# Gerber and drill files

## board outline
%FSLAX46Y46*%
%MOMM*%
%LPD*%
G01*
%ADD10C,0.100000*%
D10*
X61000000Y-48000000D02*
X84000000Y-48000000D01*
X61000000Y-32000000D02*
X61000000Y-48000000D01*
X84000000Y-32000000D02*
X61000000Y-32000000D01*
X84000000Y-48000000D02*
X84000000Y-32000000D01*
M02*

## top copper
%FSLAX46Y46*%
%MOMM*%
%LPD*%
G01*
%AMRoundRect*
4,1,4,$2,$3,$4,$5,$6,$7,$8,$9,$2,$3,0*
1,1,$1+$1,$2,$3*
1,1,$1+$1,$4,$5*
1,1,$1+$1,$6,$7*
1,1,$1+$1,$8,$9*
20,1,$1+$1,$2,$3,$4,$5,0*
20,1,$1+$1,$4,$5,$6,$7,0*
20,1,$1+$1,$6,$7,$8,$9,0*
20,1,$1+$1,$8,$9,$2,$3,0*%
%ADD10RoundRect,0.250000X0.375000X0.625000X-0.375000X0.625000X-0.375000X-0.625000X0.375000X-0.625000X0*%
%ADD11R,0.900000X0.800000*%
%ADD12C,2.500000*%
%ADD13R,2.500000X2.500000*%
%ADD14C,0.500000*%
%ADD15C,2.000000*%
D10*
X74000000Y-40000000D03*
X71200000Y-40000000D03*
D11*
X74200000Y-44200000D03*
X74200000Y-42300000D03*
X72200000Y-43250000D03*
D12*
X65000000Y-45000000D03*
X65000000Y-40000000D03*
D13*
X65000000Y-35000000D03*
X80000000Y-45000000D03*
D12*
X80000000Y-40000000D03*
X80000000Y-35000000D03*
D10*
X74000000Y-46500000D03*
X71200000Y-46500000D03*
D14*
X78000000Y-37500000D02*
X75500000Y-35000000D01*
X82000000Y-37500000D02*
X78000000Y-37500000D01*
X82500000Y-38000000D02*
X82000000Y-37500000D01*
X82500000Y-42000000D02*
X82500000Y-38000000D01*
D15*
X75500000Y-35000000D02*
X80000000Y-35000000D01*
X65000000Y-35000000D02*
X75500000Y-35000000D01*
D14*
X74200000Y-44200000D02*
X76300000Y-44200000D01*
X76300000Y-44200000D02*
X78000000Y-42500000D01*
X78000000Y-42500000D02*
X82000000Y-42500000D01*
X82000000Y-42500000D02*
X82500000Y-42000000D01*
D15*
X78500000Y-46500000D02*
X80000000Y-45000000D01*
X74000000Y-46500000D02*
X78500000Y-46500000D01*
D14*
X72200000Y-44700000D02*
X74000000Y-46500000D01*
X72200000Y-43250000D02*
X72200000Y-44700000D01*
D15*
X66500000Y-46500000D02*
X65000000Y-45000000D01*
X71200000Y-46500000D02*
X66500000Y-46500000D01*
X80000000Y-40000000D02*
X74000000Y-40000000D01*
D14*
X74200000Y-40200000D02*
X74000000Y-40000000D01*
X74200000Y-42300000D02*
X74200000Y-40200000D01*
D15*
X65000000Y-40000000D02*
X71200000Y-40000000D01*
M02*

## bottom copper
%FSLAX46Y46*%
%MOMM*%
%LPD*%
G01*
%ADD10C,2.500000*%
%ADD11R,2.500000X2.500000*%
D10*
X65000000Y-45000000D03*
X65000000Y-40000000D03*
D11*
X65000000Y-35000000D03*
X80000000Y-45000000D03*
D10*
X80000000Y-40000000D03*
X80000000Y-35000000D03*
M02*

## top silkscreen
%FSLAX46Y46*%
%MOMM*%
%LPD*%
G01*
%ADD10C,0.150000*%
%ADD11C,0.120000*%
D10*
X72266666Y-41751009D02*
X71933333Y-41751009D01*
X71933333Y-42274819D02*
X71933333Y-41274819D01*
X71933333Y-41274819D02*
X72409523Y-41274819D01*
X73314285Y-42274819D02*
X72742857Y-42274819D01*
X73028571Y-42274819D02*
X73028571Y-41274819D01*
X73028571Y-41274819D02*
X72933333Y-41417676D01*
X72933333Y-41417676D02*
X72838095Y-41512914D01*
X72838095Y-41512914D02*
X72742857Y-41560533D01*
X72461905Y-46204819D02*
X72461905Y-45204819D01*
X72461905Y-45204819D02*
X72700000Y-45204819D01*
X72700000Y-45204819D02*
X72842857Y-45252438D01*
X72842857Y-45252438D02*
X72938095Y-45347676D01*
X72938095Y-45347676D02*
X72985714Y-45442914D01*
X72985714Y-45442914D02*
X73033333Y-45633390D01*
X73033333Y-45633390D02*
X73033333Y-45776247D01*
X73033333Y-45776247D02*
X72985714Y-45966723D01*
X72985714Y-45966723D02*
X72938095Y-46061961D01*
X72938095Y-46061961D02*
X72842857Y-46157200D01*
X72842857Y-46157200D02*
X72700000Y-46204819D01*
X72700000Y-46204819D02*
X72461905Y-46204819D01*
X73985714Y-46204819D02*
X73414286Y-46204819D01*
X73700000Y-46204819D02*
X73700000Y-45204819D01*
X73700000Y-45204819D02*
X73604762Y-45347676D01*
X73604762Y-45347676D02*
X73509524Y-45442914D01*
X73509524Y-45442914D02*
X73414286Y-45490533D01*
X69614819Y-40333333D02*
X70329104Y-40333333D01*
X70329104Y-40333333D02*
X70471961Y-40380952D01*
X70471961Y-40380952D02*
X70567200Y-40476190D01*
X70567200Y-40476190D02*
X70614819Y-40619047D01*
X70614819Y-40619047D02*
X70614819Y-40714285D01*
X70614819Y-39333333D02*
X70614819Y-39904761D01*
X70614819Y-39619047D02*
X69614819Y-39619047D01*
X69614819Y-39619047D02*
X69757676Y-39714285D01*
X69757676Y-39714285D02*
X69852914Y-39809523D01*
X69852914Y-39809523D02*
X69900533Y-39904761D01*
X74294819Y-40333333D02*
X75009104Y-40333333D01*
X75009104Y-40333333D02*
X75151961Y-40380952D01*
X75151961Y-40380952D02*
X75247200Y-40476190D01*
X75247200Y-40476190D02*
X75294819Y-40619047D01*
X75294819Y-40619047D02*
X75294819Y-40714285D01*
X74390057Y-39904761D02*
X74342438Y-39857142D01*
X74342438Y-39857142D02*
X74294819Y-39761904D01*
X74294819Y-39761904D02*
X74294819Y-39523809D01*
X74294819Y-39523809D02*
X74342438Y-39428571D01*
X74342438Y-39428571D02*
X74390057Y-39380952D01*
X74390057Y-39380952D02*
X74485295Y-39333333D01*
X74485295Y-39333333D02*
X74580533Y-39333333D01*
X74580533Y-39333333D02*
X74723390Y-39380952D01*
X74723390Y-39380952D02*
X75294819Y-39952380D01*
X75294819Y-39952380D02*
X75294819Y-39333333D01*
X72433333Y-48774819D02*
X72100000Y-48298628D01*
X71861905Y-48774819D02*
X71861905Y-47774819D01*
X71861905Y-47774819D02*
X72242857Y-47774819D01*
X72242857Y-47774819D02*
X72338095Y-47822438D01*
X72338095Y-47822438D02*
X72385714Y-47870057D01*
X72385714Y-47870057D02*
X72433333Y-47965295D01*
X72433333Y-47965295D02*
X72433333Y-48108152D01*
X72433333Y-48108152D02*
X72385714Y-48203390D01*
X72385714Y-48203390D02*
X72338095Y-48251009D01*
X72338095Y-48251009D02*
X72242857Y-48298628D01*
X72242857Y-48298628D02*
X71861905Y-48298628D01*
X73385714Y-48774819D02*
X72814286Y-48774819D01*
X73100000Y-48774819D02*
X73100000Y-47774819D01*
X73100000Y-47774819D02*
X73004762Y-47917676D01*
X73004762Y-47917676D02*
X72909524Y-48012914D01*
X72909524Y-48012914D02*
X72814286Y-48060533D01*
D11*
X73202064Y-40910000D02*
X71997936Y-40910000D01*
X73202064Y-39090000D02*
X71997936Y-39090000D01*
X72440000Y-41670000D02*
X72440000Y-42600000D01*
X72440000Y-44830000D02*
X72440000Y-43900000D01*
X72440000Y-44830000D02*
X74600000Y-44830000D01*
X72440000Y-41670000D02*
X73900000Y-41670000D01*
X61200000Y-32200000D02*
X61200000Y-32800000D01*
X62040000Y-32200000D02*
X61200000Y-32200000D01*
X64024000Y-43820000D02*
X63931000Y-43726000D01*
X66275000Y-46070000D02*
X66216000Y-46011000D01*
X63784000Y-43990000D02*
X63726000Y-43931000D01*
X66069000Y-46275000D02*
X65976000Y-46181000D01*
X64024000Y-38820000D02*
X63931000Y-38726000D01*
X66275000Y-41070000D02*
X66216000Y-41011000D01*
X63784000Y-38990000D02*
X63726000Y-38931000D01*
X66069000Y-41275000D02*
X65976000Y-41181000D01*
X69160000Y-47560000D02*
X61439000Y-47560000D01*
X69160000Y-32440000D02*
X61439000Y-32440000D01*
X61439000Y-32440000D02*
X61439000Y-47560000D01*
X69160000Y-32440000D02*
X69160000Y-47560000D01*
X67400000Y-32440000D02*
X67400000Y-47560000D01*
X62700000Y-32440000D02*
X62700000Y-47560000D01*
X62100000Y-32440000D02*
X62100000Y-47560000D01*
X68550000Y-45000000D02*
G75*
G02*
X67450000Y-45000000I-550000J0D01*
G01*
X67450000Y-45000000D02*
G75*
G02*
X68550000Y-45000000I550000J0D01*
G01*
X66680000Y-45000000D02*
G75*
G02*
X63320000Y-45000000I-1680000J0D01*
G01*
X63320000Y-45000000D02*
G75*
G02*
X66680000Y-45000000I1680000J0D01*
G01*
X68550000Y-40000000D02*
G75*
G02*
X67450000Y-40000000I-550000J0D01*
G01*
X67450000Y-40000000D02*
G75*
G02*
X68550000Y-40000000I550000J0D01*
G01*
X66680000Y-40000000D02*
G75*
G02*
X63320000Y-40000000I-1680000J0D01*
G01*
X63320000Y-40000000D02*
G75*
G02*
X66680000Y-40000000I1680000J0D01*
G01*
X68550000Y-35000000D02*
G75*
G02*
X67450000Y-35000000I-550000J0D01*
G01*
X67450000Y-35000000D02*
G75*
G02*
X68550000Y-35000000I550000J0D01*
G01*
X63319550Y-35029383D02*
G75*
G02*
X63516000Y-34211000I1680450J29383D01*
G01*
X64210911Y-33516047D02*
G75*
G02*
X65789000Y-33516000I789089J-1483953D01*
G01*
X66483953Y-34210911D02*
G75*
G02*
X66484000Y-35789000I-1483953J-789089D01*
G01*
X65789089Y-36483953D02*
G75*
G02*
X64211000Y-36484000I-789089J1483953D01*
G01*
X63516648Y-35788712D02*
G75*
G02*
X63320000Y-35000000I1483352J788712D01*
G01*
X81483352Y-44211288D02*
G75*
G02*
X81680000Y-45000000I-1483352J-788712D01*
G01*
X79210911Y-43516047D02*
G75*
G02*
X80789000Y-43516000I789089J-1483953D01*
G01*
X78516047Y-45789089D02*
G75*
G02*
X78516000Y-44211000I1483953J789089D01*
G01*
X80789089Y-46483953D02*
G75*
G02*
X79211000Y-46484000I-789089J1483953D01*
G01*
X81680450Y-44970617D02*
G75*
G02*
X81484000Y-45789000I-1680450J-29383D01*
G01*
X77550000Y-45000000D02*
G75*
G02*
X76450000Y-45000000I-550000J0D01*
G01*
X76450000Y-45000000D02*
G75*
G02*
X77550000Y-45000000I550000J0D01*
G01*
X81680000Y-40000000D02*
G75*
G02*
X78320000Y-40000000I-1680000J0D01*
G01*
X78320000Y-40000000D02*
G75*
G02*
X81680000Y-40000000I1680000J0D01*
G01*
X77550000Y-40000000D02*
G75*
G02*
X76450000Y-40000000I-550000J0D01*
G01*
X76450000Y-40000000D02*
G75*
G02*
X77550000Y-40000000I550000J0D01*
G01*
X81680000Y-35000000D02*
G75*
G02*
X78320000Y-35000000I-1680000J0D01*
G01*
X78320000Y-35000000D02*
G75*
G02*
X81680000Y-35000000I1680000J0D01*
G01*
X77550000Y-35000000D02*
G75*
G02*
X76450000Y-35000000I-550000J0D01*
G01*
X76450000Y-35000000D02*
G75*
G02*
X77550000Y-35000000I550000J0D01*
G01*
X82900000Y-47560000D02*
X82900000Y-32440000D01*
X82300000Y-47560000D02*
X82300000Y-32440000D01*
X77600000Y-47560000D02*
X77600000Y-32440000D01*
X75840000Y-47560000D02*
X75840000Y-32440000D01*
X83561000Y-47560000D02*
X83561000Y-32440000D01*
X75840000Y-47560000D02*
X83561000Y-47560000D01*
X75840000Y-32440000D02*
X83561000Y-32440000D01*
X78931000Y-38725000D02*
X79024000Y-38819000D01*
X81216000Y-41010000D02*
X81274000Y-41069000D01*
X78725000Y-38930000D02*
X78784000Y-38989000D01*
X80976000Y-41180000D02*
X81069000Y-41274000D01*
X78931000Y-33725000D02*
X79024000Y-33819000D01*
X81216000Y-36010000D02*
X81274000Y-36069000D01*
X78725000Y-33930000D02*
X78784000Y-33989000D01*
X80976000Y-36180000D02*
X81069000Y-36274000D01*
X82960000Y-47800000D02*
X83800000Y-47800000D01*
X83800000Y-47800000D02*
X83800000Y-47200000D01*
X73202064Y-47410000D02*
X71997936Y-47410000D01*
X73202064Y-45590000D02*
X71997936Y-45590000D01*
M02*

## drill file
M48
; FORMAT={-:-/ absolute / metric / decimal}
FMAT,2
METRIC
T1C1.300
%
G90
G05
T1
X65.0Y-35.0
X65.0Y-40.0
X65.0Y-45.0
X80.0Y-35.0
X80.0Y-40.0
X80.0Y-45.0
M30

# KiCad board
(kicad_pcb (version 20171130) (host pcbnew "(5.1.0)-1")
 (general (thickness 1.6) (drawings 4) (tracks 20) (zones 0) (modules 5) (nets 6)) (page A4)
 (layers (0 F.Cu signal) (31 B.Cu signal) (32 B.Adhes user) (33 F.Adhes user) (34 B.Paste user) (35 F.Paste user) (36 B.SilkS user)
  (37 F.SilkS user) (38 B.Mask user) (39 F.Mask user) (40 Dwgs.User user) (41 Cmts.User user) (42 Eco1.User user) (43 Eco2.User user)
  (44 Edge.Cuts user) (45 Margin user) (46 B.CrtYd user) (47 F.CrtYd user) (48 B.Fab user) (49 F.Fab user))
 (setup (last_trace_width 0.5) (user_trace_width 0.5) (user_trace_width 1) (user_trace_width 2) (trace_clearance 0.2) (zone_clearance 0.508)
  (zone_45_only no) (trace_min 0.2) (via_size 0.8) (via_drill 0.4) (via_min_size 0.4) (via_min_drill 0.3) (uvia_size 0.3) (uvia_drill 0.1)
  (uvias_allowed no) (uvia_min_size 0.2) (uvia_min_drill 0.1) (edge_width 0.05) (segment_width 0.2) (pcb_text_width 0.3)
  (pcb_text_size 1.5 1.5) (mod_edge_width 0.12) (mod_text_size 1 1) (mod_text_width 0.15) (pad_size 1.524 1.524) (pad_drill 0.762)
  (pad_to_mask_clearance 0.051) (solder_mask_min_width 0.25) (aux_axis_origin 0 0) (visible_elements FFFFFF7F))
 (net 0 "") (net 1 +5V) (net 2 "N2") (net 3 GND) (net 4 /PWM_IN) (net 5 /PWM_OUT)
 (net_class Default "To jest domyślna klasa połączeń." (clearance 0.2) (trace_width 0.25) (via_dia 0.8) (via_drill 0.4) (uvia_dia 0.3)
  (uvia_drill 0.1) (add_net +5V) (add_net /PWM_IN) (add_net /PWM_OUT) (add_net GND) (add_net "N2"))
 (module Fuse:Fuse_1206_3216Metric (layer F.Cu) (at 72.6 40 180)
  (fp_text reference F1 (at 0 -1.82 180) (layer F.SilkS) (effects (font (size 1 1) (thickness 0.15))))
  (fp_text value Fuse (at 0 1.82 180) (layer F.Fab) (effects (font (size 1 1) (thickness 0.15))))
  (fp_line (start -0.602064 -0.91) (end 0.602064 -0.91) (layer F.SilkS) (width 0.12))
  (fp_line (start -0.602064 0.91) (end 0.602064 0.91) (layer F.SilkS) (width 0.12))
  (pad 1 smd roundrect (at -1.4 0 180) (size 1.25 1.75) (layers F.Cu F.Paste F.Mask) (roundrect_rratio 0.2) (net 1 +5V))
  (pad 2 smd roundrect (at 1.4 0 180) (size 1.25 1.75) (layers F.Cu F.Paste F.Mask) (roundrect_rratio 0.2) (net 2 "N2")))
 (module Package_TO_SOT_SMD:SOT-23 (layer F.Cu) (at 73.2 43.25 180)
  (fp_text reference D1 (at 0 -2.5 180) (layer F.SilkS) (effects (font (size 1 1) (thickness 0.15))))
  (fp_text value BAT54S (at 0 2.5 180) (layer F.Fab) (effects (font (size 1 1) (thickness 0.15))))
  (fp_line (start 0.76 1.58) (end 0.76 0.65) (layer F.SilkS) (width 0.12))
  (fp_line (start 0.76 -1.58) (end 0.76 -0.65) (layer F.SilkS) (width 0.12))
  (fp_line (start 0.76 -1.58) (end -1.4 -1.58) (layer F.SilkS) (width 0.12))
  (fp_line (start 0.76 1.58) (end -0.7 1.58) (layer F.SilkS) (width 0.12))
  (pad 1 smd rect (at -1 -0.95 180) (size 0.9 0.8) (layers F.Cu F.Paste F.Mask) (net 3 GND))
  (pad 2 smd rect (at -1 0.95 180) (size 0.9 0.8) (layers F.Cu F.Paste F.Mask) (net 1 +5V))
  (pad 3 smd rect (at 1 0 180) (size 0.9 0.8) (layers F.Cu F.Paste F.Mask) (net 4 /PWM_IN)))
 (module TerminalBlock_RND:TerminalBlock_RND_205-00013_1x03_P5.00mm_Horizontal (layer F.Cu) (at 65 35 270)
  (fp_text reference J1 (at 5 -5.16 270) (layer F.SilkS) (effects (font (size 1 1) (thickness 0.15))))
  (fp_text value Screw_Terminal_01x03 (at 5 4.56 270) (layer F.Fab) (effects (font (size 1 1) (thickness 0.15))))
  (fp_line (start -2.8 3.8) (end -2.2 3.8) (layer F.SilkS) (width 0.12))
  (fp_line (start -2.8 2.96) (end -2.8 3.8) (layer F.SilkS) (width 0.12))
  (fp_line (start 8.82 0.976) (end 8.726 1.069) (layer F.SilkS) (width 0.12))
  (fp_line (start 11.07 -1.275) (end 11.011 -1.216) (layer F.SilkS) (width 0.12))
  (fp_line (start 8.99 1.216) (end 8.931 1.274) (layer F.SilkS) (width 0.12))
  (fp_line (start 11.275 -1.069) (end 11.181 -0.976) (layer F.SilkS) (width 0.12))
  (fp_line (start 3.82 0.976) (end 3.726 1.069) (layer F.SilkS) (width 0.12))
  (fp_line (start 6.07 -1.275) (end 6.011 -1.216) (layer F.SilkS) (width 0.12))
  (fp_line (start 3.99 1.216) (end 3.931 1.274) (layer F.SilkS) (width 0.12))
  (fp_line (start 6.275 -1.069) (end 6.181 -0.976) (layer F.SilkS) (width 0.12))
  (fp_line (start 12.56 -4.16) (end 12.56 3.561) (layer F.SilkS) (width 0.12))
  (fp_line (start -2.56 -4.16) (end -2.56 3.561) (layer F.SilkS) (width 0.12))
  (fp_line (start -2.56 3.561) (end 12.56 3.561) (layer F.SilkS) (width 0.12))
  (fp_line (start -2.56 -4.16) (end 12.56 -4.16) (layer F.SilkS) (width 0.12))
  (fp_line (start -2.56 -2.4) (end 12.56 -2.4) (layer F.SilkS) (width 0.12))
  (fp_line (start -2.56 2.3) (end 12.56 2.3) (layer F.SilkS) (width 0.12))
  (fp_line (start -2.56 2.9) (end 12.56 2.9) (layer F.SilkS) (width 0.12))
  (fp_circle (center 10 -3) (end 10.55 -3) (layer F.SilkS) (width 0.12))
  (fp_circle (center 10 0) (end 11.68 0) (layer F.SilkS) (width 0.12))
  (fp_circle (center 5 -3) (end 5.55 -3) (layer F.SilkS) (width 0.12))
  (fp_circle (center 5 0) (end 6.68 0) (layer F.SilkS) (width 0.12))
  (fp_circle (center 0 -3) (end 0.55 -3) (layer F.SilkS) (width 0.12))
  (fp_arc (start 0 0) (end -0.789 1.484) (angle -29) (layer F.SilkS) (width 0.12))
  (fp_arc (start 0 0) (end -1.484 -0.789) (angle -56) (layer F.SilkS) (width 0.12))
  (fp_arc (start 0 0) (end 0.789 -1.484) (angle -56) (layer F.SilkS) (width 0.12))
  (fp_arc (start 0 0) (end 1.484 0.789) (angle -56) (layer F.SilkS) (width 0.12))
  (fp_arc (start 0 0) (end 0 1.68) (angle -28) (layer F.SilkS) (width 0.12))
  (pad 3 thru_hole circle (at 10 0 270) (size 2.5 2.5) (drill 1.3) (layers *.Cu *.Mask) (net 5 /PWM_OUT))
  (pad 2 thru_hole circle (at 5 0 270) (size 2.5 2.5) (drill 1.3) (layers *.Cu *.Mask) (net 2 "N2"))
  (pad 1 thru_hole rect (at 0 0 270) (size 2.5 2.5) (drill 1.3) (layers *.Cu *.Mask) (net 3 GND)))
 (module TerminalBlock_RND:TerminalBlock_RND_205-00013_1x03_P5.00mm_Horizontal (layer F.Cu) (at 80 45 90)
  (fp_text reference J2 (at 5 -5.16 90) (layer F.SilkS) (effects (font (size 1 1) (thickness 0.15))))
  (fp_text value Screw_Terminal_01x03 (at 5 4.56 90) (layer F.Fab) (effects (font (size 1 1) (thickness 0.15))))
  (fp_arc (start 0 0) (end 0 1.68) (angle -28) (layer F.SilkS) (width 0.12))
  (fp_arc (start 0 0) (end 1.484 0.789) (angle -56) (layer F.SilkS) (width 0.12))
  (fp_arc (start 0 0) (end 0.789 -1.484) (angle -56) (layer F.SilkS) (width 0.12))
  (fp_arc (start 0 0) (end -1.484 -0.789) (angle -56) (layer F.SilkS) (width 0.12))
  (fp_arc (start 0 0) (end -0.789 1.484) (angle -29) (layer F.SilkS) (width 0.12))
  (fp_circle (center 0 -3) (end 0.55 -3) (layer F.SilkS) (width 0.12))
  (fp_circle (center 5 0) (end 6.68 0) (layer F.SilkS) (width 0.12))
  (fp_circle (center 5 -3) (end 5.55 -3) (layer F.SilkS) (width 0.12))
  (fp_circle (center 10 0) (end 11.68 0) (layer F.SilkS) (width 0.12))
  (fp_circle (center 10 -3) (end 10.55 -3) (layer F.SilkS) (width 0.12))
  (fp_line (start -2.56 2.9) (end 12.56 2.9) (layer F.SilkS) (width 0.12))
  (fp_line (start -2.56 2.3) (end 12.56 2.3) (layer F.SilkS) (width 0.12))
  (fp_line (start -2.56 -2.4) (end 12.56 -2.4) (layer F.SilkS) (width 0.12))
  (fp_line (start -2.56 -4.16) (end 12.56 -4.16) (layer F.SilkS) (width 0.12))
  (fp_line (start -2.56 3.561) (end 12.56 3.561) (layer F.SilkS) (width 0.12))
  (fp_line (start -2.56 -4.16) (end -2.56 3.561) (layer F.SilkS) (width 0.12))
  (fp_line (start 12.56 -4.16) (end 12.56 3.561) (layer F.SilkS) (width 0.12))
  (fp_line (start 6.275 -1.069) (end 6.181 -0.976) (layer F.SilkS) (width 0.12))
  (fp_line (start 3.99 1.216) (end 3.931 1.274) (layer F.SilkS) (width 0.12))
  (fp_line (start 6.07 -1.275) (end 6.011 -1.216) (layer F.SilkS) (width 0.12))
  (fp_line (start 3.82 0.976) (end 3.726 1.069) (layer F.SilkS) (width 0.12))
  (fp_line (start 11.275 -1.069) (end 11.181 -0.976) (layer F.SilkS) (width 0.12))
  (fp_line (start 8.99 1.216) (end 8.931 1.274) (layer F.SilkS) (width 0.12))
  (fp_line (start 11.07 -1.275) (end 11.011 -1.216) (layer F.SilkS) (width 0.12))
  (fp_line (start 8.82 0.976) (end 8.726 1.069) (layer F.SilkS) (width 0.12))
  (fp_line (start -2.8 2.96) (end -2.8 3.8) (layer F.SilkS) (width 0.12))
  (fp_line (start -2.8 3.8) (end -2.2 3.8) (layer F.SilkS) (width 0.12))
  (pad 1 thru_hole rect (at 0 0 90) (size 2.5 2.5) (drill 1.3) (layers *.Cu *.Mask) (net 4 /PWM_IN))
  (pad 2 thru_hole circle (at 5 0 90) (size 2.5 2.5) (drill 1.3) (layers *.Cu *.Mask) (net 1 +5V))
  (pad 3 thru_hole circle (at 10 0 90) (size 2.5 2.5) (drill 1.3) (layers *.Cu *.Mask) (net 3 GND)))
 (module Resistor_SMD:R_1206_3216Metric (layer F.Cu) (at 72.6 46.5 180)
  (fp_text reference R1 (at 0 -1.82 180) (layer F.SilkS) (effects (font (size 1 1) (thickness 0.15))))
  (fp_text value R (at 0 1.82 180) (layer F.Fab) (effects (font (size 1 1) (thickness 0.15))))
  (fp_line (start -0.602064 -0.91) (end 0.602064 -0.91) (layer F.SilkS) (width 0.12))
  (fp_line (start -0.602064 0.91) (end 0.602064 0.91) (layer F.SilkS) (width 0.12))
  (pad 1 smd roundrect (at -1.4 0 180) (size 1.25 1.75) (layers F.Cu F.Paste F.Mask) (roundrect_rratio 0.2) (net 4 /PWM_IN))
  (pad 2 smd roundrect (at 1.4 0 180) (size 1.25 1.75) (layers F.Cu F.Paste F.Mask) (roundrect_rratio 0.2) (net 5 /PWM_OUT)))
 (gr_line (start 61 48) (end 84 48) (layer Edge.Cuts) (width 0.1))
 (gr_line (start 61 32) (end 61 48) (layer Edge.Cuts) (width 0.1))
 (gr_line (start 84 32) (end 61 32) (layer Edge.Cuts) (width 0.1))
 (gr_line (start 84 48) (end 84 32) (layer Edge.Cuts) (width 0.1))
 (segment (start 78 37.5) (end 75.5 35) (width 0.5) (layer F.Cu) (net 3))
 (segment (start 82 37.5) (end 78 37.5) (width 0.5) (layer F.Cu) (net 3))
 (segment (start 82.5 38) (end 82 37.5) (width 0.5) (layer F.Cu) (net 3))
 (segment (start 82.5 42) (end 82.5 38) (width 0.5) (layer F.Cu) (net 3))
 (segment (start 75.5 35) (end 80 35) (width 2) (layer F.Cu) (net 3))
 (segment (start 65 35) (end 75.5 35) (width 2) (layer F.Cu) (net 3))
 (segment (start 74.2 44.2) (end 76.3 44.2) (width 0.5) (layer F.Cu) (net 3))
 (segment (start 76.3 44.2) (end 78 42.5) (width 0.5) (layer F.Cu) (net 3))
 (segment (start 78 42.5) (end 82 42.5) (width 0.5) (layer F.Cu) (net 3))
 (segment (start 82 42.5) (end 82.5 42) (width 0.5) (layer F.Cu) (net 3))
 (segment (start 78.5 46.5) (end 80 45) (width 2) (layer F.Cu) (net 4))
 (segment (start 74 46.5) (end 78.5 46.5) (width 2) (layer F.Cu) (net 4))
 (segment (start 72.2 44.7) (end 74 46.5) (width 0.5) (layer F.Cu) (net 4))
 (segment (start 72.2 43.25) (end 72.2 44.7) (width 0.5) (layer F.Cu) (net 4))
 (segment (start 66.5 46.5) (end 65 45) (width 2) (layer F.Cu) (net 5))
 (segment (start 71.2 46.5) (end 66.5 46.5) (width 2) (layer F.Cu) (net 5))
 (segment (start 80 40) (end 74 40) (width 2) (layer F.Cu) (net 1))
 (segment (start 74.2 40.2) (end 74 40) (width 0.5) (layer F.Cu) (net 1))
 (segment (start 74.2 42.3) (end 74.2 40.2) (width 0.5) (layer F.Cu) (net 1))
 (segment (start 65 40) (end 71.2 40) (width 2) (layer F.Cu) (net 2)))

